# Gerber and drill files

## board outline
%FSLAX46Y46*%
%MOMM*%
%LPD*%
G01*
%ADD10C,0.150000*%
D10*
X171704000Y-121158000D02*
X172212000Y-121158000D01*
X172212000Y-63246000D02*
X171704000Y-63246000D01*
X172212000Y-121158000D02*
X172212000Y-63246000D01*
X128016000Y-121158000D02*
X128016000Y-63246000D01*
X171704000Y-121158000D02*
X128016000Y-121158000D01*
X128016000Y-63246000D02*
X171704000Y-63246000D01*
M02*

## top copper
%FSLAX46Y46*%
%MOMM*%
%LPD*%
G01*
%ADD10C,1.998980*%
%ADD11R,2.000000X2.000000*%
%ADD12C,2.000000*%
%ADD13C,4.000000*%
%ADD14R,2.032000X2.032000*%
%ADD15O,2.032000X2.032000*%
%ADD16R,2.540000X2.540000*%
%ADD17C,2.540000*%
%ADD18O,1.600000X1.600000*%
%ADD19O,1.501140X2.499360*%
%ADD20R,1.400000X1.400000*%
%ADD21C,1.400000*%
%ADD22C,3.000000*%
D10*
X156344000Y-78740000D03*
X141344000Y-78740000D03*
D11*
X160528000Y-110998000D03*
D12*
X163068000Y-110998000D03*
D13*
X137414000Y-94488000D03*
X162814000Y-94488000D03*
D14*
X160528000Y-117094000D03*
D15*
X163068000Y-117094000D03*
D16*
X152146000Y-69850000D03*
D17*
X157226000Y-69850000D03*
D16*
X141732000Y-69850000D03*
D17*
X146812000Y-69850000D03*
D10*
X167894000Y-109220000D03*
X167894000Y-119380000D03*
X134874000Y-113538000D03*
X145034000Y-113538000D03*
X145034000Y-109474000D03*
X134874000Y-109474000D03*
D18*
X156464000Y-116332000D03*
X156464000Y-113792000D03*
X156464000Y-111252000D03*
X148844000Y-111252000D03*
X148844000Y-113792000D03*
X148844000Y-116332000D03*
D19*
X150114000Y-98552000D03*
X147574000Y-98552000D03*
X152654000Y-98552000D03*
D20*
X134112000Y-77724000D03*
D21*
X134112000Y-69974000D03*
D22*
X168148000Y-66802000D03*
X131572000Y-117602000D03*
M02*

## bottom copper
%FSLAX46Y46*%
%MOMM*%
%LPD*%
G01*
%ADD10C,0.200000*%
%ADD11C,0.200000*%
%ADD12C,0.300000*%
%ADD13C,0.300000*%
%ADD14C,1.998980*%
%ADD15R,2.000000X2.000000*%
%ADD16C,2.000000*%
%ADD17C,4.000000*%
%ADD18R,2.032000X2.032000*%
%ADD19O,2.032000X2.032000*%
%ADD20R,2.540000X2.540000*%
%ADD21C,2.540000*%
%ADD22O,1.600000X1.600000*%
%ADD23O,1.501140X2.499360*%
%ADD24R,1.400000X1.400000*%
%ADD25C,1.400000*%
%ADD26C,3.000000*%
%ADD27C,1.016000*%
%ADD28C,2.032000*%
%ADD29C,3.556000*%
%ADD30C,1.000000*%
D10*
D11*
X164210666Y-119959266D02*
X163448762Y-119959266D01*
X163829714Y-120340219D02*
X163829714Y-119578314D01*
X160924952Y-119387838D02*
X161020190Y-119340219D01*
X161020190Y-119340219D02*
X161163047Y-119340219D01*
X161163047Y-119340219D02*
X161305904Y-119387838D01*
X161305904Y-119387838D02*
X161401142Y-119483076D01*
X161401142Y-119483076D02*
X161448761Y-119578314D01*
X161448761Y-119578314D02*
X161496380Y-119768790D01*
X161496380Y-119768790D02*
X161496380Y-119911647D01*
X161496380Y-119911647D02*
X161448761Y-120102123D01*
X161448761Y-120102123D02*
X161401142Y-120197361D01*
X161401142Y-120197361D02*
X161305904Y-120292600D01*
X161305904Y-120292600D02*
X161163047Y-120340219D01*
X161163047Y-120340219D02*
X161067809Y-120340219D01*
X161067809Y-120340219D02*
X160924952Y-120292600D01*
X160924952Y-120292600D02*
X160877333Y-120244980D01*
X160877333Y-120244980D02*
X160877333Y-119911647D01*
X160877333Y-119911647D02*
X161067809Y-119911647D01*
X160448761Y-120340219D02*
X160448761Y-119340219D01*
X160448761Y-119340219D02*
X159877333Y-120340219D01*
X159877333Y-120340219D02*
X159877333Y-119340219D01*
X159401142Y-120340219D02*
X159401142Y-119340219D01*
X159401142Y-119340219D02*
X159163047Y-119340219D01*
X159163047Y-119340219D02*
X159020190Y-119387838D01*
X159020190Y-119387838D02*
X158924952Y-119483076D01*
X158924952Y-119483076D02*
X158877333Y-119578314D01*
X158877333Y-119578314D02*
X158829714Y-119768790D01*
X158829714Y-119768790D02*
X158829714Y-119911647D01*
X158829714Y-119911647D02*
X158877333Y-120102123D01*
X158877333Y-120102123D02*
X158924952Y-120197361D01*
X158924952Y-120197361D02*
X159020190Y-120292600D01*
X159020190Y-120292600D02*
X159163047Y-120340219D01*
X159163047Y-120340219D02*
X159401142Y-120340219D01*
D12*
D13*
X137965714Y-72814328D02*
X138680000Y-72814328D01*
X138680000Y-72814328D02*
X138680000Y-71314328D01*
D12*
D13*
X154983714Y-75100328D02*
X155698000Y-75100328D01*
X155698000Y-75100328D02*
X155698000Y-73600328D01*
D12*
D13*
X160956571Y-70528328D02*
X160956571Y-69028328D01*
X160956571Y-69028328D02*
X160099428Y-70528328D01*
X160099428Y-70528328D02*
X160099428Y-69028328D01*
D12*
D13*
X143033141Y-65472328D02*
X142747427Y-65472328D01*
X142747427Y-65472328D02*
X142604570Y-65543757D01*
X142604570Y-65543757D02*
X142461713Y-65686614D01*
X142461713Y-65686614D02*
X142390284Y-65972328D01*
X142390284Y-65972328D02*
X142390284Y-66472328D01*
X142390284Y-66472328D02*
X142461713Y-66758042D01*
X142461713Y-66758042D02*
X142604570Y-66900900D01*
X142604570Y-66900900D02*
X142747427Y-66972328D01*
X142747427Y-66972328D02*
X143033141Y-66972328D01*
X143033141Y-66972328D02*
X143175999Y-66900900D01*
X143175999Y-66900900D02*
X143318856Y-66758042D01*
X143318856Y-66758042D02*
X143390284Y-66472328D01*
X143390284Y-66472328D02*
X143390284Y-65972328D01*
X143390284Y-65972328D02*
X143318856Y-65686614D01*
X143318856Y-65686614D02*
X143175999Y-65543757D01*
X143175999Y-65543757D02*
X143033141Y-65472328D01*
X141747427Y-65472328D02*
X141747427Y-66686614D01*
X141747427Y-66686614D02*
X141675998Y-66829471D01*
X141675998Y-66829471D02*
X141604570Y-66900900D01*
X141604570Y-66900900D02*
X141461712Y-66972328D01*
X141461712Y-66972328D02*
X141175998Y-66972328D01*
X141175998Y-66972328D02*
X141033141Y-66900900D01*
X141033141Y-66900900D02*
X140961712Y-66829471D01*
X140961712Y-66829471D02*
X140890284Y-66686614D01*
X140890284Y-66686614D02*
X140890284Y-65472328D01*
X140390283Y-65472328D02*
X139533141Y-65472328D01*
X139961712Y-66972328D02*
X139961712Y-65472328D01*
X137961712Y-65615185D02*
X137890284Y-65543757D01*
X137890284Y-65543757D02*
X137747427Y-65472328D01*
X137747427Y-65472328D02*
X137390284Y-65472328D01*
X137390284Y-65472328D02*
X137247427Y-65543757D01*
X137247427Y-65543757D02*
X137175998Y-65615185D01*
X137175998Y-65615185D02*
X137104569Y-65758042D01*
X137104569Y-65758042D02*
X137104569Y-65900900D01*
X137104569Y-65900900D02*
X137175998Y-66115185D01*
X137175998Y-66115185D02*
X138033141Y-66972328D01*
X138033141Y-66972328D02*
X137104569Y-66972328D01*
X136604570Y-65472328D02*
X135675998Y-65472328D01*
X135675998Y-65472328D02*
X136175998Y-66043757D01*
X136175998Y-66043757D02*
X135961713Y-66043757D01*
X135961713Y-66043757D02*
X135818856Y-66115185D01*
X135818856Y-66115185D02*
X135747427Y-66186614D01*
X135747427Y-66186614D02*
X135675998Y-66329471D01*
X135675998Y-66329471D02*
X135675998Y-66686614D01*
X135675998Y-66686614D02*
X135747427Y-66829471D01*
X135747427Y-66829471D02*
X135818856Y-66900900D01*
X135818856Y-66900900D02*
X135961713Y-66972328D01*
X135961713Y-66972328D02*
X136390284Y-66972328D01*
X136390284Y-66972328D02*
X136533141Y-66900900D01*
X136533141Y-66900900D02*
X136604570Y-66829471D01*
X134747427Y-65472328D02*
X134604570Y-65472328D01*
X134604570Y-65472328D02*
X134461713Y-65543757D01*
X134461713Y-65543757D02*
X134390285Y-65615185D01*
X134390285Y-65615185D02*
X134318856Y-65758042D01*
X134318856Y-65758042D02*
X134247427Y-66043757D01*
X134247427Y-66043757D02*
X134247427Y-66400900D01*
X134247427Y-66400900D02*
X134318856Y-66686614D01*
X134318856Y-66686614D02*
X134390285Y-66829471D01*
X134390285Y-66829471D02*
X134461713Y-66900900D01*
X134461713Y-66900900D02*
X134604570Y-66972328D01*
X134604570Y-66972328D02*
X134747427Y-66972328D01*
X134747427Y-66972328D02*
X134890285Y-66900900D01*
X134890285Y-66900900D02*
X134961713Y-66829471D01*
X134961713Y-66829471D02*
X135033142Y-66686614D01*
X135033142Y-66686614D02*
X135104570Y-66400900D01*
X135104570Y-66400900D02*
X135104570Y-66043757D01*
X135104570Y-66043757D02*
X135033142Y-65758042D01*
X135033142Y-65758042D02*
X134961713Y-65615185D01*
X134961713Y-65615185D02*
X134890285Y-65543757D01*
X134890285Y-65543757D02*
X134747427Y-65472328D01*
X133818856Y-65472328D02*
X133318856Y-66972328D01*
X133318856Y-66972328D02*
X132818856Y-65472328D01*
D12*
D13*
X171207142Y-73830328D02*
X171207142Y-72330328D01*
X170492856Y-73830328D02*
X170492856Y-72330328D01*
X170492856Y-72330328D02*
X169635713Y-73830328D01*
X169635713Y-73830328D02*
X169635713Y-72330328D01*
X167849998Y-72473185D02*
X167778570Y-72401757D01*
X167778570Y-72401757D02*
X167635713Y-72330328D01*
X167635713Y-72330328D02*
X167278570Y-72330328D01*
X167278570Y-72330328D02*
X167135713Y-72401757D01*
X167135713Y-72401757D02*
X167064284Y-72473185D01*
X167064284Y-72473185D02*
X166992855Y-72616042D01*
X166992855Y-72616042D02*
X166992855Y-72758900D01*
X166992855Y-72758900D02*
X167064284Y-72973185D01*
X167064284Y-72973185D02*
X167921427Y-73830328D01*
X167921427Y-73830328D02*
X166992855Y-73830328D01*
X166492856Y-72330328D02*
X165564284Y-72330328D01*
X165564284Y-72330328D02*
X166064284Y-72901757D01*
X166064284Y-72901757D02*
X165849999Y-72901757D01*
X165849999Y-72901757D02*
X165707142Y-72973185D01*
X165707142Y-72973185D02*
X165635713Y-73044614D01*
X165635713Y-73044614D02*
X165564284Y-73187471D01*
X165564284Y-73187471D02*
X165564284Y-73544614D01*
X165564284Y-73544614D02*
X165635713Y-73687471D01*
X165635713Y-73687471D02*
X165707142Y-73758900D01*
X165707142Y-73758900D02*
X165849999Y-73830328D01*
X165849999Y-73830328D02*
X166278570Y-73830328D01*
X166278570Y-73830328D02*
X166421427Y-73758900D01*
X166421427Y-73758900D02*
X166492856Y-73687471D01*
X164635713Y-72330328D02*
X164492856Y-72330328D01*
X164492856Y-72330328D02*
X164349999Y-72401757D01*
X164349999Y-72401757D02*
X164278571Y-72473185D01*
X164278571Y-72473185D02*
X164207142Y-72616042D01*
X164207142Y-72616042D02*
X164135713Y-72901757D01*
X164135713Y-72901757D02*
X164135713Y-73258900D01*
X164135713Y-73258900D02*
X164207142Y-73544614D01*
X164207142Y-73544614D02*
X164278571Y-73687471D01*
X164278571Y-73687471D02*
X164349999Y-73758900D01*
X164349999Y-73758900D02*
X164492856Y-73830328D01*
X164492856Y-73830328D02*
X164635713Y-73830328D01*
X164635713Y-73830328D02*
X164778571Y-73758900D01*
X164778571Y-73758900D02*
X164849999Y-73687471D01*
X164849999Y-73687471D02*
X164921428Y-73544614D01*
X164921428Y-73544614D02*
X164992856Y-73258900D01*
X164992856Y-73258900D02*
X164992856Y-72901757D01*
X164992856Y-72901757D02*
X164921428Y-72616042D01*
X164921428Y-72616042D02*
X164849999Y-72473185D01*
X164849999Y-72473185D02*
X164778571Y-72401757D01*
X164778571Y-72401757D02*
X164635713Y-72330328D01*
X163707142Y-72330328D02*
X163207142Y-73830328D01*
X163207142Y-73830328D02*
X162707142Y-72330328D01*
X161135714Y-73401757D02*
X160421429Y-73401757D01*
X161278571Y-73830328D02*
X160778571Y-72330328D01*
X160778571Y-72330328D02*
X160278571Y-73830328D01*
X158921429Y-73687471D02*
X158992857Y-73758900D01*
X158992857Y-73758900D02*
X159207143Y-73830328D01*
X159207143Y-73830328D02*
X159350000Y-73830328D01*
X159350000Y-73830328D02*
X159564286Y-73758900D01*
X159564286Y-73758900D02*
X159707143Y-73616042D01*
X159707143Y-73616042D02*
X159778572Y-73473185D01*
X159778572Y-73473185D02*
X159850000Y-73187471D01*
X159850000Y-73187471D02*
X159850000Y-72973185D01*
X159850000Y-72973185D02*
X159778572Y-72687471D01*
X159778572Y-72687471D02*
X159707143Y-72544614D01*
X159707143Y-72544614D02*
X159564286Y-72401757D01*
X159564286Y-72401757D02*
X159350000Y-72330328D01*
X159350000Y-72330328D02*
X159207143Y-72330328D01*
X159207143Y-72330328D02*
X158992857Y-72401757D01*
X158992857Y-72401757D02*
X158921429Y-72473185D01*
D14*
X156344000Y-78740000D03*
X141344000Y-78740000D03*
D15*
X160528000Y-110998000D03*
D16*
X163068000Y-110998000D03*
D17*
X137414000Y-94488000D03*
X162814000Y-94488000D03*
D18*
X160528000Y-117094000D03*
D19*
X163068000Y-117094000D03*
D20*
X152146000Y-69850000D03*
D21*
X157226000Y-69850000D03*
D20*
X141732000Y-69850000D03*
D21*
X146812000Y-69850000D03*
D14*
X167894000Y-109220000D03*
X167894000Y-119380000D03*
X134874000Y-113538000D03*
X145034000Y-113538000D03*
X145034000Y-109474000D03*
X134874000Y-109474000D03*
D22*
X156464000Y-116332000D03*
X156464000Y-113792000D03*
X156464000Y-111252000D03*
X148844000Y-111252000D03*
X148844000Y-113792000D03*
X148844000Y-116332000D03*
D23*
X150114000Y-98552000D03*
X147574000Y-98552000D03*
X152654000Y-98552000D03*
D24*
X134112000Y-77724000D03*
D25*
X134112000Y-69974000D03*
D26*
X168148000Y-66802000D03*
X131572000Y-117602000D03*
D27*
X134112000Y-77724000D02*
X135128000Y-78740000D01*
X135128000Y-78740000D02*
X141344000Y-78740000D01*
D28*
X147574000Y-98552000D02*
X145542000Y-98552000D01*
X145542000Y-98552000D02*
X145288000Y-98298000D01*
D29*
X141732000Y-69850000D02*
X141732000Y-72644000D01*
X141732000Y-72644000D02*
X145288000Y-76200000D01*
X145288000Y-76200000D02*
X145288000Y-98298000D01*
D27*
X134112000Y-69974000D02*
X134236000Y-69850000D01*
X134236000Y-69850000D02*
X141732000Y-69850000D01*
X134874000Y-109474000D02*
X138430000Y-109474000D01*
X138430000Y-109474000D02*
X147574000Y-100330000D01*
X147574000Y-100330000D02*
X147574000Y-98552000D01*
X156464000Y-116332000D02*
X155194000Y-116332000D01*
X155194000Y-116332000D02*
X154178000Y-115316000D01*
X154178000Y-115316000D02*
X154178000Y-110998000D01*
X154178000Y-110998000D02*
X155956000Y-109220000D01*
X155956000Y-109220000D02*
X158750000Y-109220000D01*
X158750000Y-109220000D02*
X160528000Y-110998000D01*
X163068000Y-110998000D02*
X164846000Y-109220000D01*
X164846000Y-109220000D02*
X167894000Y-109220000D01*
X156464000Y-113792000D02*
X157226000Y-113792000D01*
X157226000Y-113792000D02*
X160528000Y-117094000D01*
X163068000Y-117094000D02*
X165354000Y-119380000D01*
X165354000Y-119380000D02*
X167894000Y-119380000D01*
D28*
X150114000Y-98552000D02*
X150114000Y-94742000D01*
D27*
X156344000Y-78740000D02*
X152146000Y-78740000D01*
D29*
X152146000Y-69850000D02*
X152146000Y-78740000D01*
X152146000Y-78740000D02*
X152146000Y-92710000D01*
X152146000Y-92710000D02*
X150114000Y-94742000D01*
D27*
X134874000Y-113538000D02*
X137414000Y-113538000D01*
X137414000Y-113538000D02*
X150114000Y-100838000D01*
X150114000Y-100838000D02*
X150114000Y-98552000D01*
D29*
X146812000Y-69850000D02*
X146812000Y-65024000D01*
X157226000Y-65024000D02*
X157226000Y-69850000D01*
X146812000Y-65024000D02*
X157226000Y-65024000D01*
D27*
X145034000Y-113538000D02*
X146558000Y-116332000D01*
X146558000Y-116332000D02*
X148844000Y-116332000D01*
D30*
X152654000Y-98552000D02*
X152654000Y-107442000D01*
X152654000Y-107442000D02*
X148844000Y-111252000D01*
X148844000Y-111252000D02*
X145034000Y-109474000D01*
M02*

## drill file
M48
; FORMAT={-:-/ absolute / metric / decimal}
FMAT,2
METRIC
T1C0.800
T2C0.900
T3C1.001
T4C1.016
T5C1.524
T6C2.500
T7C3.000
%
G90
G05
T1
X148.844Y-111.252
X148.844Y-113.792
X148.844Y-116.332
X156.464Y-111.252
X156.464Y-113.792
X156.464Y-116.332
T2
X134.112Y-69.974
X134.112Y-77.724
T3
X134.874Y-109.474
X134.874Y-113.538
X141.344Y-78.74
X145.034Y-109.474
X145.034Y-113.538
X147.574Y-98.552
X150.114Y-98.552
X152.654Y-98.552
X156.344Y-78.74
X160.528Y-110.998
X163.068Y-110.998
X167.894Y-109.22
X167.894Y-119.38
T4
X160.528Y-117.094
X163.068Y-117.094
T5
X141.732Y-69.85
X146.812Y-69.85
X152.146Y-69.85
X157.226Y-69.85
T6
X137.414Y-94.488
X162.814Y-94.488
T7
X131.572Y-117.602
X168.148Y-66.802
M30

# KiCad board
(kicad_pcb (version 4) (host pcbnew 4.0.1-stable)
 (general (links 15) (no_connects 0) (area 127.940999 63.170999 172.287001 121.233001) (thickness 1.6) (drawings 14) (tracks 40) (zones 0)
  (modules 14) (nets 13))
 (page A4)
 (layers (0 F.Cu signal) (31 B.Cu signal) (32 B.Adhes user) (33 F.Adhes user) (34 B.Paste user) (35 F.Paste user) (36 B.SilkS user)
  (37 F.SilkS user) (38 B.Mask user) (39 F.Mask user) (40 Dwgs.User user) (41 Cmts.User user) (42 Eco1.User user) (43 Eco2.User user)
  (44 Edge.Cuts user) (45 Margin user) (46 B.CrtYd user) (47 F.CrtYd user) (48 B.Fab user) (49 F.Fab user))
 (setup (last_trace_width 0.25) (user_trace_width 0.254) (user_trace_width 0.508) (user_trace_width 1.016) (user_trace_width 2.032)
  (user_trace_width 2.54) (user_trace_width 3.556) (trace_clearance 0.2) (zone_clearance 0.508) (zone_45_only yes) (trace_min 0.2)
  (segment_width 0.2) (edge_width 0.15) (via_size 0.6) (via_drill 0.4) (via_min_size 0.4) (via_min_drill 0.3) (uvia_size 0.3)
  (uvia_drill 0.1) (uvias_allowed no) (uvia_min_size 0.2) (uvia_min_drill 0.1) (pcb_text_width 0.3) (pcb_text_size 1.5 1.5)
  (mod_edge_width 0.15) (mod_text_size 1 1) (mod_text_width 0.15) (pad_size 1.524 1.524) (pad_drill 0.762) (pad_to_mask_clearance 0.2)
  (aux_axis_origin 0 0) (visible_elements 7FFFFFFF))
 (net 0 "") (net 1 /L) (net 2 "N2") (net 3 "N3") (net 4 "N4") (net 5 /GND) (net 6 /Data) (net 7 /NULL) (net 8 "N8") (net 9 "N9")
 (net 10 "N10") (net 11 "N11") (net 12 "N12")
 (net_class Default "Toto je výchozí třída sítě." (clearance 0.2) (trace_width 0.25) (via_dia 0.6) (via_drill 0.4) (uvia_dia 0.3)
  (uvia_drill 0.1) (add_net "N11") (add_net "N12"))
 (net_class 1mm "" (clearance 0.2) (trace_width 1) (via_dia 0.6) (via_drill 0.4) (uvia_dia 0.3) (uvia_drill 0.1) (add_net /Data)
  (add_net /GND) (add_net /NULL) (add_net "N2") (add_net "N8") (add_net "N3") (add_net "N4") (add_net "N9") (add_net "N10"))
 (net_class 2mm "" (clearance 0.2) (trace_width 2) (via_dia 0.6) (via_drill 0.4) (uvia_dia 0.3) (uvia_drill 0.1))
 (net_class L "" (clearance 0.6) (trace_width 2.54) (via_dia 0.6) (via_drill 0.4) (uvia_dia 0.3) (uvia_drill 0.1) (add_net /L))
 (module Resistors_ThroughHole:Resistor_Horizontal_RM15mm (layer F.Cu) (at 148.844 78.74 180)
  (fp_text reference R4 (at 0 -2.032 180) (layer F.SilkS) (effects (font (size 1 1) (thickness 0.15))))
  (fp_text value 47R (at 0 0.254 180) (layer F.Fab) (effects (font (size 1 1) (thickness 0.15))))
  (pad 1 thru_hole circle (at -7.5 0 180) (size 1.99898 1.99898) (drill 1.00076) (layers *.Cu *.SilkS *.Mask) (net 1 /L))
  (pad 2 thru_hole circle (at 7.5 0 180) (size 1.99898 1.99898) (drill 1.00076) (layers *.Cu *.SilkS *.Mask) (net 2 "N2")))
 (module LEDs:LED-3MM (layer F.Cu) (at 160.528 110.998)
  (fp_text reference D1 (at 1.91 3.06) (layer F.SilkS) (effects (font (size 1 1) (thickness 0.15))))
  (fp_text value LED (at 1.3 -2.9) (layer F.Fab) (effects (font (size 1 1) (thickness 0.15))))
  (pad 1 thru_hole rect (at 0 0 90) (size 2 2) (drill 1.00076) (layers *.Cu *.Mask F.SilkS) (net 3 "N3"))
  (pad 2 thru_hole circle (at 2.54 0) (size 2 2) (drill 1.00076) (layers *.Cu *.Mask F.SilkS) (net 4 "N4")))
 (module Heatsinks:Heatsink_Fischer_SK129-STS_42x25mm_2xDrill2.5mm (layer F.Cu) (at 150.114 94.488)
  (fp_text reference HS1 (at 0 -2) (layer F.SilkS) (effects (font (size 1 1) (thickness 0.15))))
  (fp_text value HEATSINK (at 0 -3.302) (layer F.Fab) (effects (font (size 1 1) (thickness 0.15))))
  (pad 1 thru_hole circle (at -12.7 0) (size 4 4) (drill 2.5) (layers *.Cu *.Mask F.SilkS))
  (pad 1 thru_hole circle (at 12.7 0) (size 4 4) (drill 2.5) (layers *.Cu *.Mask F.SilkS)))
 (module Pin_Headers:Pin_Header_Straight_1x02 (layer F.Cu) (at 160.528 117.094 90)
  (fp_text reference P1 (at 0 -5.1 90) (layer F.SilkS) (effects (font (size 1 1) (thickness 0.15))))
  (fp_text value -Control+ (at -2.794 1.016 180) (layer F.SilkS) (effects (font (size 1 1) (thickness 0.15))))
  (pad 1 thru_hole rect (at 0 0 90) (size 2.032 2.032) (drill 1.016) (layers *.Cu *.Mask F.SilkS) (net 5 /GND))
  (pad 2 thru_hole oval (at 0 2.54 90) (size 2.032 2.032) (drill 1.016) (layers *.Cu *.Mask F.SilkS) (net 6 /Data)))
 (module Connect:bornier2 (layer F.Cu) (at 154.686 69.85)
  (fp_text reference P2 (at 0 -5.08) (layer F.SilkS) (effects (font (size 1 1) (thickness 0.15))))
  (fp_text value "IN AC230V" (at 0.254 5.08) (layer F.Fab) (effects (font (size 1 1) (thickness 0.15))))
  (pad 1 thru_hole rect (at -2.54 0) (size 2.54 2.54) (drill 1.524) (layers *.Cu *.Mask F.SilkS) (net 1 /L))
  (pad 2 thru_hole circle (at 2.54 0) (size 2.54 2.54) (drill 1.524) (layers *.Cu *.Mask F.SilkS) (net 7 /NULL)))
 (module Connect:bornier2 (layer F.Cu) (at 144.272 69.85)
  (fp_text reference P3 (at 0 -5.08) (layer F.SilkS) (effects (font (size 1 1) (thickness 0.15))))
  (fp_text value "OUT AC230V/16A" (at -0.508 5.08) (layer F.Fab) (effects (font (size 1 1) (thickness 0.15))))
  (pad 1 thru_hole rect (at -2.54 0) (size 2.54 2.54) (drill 1.524) (layers *.Cu *.Mask F.SilkS) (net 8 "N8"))
  (pad 2 thru_hole circle (at 2.54 0) (size 2.54 2.54) (drill 1.524) (layers *.Cu *.Mask F.SilkS) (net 7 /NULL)))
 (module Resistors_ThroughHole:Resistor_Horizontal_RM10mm (layer F.Cu) (at 167.894 114.3 270)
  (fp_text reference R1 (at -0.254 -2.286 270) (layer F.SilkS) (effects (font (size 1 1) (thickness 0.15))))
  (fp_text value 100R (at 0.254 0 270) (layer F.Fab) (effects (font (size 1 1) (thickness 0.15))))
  (pad 1 thru_hole circle (at -5.08 0 270) (size 1.99898 1.99898) (drill 1.00076) (layers *.Cu *.SilkS *.Mask) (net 4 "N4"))
  (pad 2 thru_hole circle (at 5.08 0 270) (size 1.99898 1.99898) (drill 1.00076) (layers *.Cu *.SilkS *.Mask) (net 6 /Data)))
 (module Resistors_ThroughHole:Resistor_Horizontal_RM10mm (layer F.Cu) (at 139.954 113.538)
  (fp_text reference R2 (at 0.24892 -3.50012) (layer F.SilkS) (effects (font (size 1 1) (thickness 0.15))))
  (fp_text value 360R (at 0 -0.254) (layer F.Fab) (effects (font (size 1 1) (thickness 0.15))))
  (pad 1 thru_hole circle (at -5.08 0) (size 1.99898 1.99898) (drill 1.00076) (layers *.Cu *.SilkS *.Mask) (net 1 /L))
  (pad 2 thru_hole circle (at 5.08 0) (size 1.99898 1.99898) (drill 1.00076) (layers *.Cu *.SilkS *.Mask) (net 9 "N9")))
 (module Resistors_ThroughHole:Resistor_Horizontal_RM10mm (layer F.Cu) (at 139.954 109.474 180)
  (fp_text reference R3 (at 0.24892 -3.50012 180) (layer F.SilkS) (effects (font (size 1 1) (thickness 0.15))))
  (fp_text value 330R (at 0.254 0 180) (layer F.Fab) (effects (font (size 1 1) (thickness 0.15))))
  (pad 1 thru_hole circle (at -5.08 0 180) (size 1.99898 1.99898) (drill 1.00076) (layers *.Cu *.SilkS *.Mask) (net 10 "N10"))
  (pad 2 thru_hole circle (at 5.08 0 180) (size 1.99898 1.99898) (drill 1.00076) (layers *.Cu *.SilkS *.Mask) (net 8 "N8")))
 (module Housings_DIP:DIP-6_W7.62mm (layer F.Cu) (at 156.464 116.332 180)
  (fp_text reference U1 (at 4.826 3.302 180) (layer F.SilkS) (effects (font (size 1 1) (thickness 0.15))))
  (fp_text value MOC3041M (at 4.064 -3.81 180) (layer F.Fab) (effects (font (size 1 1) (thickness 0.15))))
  (pad 1 thru_hole oval (at 0 0 180) (size 1.6 1.6) (drill 0.8) (layers *.Cu *.Mask F.SilkS) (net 3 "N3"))
  (pad 2 thru_hole oval (at 0 2.54 180) (size 1.6 1.6) (drill 0.8) (layers *.Cu *.Mask F.SilkS) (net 5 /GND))
  (pad 3 thru_hole oval (at 0 5.08 180) (size 1.6 1.6) (drill 0.8) (layers *.Cu *.Mask F.SilkS))
  (pad 4 thru_hole oval (at 7.62 5.08 180) (size 1.6 1.6) (drill 0.8) (layers *.Cu *.Mask F.SilkS) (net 10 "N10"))
  (pad 5 thru_hole oval (at 7.62 2.54 180) (size 1.6 1.6) (drill 0.8) (layers *.Cu *.Mask F.SilkS))
  (pad 6 thru_hole oval (at 7.62 0 180) (size 1.6 1.6) (drill 0.8) (layers *.Cu *.Mask F.SilkS) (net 9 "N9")))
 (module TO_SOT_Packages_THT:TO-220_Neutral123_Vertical (layer F.Cu) (at 150.114 98.552)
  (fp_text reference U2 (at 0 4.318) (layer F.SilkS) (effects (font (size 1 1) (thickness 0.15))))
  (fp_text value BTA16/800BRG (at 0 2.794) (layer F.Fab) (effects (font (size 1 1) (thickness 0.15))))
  (pad 2 thru_hole oval (at 0 0 90) (size 2.49936 1.50114) (drill 1.00076) (layers *.Cu *.Mask F.SilkS) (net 1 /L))
  (pad 1 thru_hole oval (at -2.54 0 90) (size 2.49936 1.50114) (drill 1.00076) (layers *.Cu *.Mask F.SilkS) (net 8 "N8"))
  (pad 3 thru_hole oval (at 2.54 0 90) (size 2.49936 1.50114) (drill 1.00076) (layers *.Cu *.Mask F.SilkS) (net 10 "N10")))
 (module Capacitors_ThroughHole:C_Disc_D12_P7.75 (layer F.Cu) (at 134.112 77.724 90)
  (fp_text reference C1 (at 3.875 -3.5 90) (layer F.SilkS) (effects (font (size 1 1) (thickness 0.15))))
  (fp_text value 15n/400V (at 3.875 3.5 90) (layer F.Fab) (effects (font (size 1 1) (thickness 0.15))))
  (pad 1 thru_hole rect (at 0 0 90) (size 1.4 1.4) (drill 0.9) (layers *.Cu *.Mask F.SilkS) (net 2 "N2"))
  (pad 2 thru_hole circle (at 7.75 0 90) (size 1.4 1.4) (drill 0.9) (layers *.Cu *.Mask F.SilkS) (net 8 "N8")))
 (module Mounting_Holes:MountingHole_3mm (layer F.Cu) (at 168.148 66.802)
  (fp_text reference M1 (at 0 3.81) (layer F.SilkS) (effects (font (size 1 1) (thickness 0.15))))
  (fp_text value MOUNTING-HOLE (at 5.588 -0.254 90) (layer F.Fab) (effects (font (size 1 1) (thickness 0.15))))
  (pad 1 thru_hole circle (at 0 0) (size 3 3) (drill 3) (layers) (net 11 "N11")))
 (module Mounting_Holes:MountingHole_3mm (layer F.Cu) (at 131.572 117.602)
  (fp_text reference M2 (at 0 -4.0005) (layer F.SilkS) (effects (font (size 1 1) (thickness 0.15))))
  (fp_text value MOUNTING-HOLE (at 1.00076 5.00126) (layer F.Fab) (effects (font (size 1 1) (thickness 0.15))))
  (pad 1 thru_hole circle (at 0 0) (size 3 3) (drill 3) (layers) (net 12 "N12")))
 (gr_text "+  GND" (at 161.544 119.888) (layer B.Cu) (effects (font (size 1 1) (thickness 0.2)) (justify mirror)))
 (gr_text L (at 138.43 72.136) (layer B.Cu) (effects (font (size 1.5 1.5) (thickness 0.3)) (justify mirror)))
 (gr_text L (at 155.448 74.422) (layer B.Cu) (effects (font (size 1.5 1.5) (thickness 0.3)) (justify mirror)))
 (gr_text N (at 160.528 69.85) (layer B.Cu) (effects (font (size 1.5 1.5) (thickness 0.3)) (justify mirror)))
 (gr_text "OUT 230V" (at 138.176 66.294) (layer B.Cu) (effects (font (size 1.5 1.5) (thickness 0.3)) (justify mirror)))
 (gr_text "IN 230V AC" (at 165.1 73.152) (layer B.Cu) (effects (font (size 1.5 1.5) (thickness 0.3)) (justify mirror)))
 (gr_line (start 171.704 121.158) (end 172.212 121.158) (angle 90) (layer Edge.Cuts) (width 0.15))
 (gr_line (start 172.212 63.246) (end 171.704 63.246) (angle 90) (layer Edge.Cuts) (width 0.15))
 (gr_line (start 172.212 121.158) (end 172.212 63.246) (angle 90) (layer Edge.Cuts) (width 0.15))
 (gr_line (start 128.016 121.158) (end 128.016 63.246) (angle 90) (layer Edge.Cuts) (width 0.15))
 (gr_line (start 171.704 121.158) (end 128.016 121.158) (angle 90) (layer Edge.Cuts) (width 0.15))
 (gr_line (start 128.016 63.246) (end 171.704 63.246) (angle 90) (layer Edge.Cuts) (width 0.15))
 (segment (start 134.112 77.724) (end 135.128 78.74) (width 1.016) (layer B.Cu) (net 2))
 (segment (start 135.128 78.74) (end 141.344 78.74) (width 1.016) (layer B.Cu) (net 2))
 (segment (start 147.574 98.552) (end 145.542 98.552) (width 2.032) (layer B.Cu) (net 8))
 (segment (start 145.542 98.552) (end 145.288 98.298) (width 2.032) (layer B.Cu) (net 8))
 (segment (start 141.732 69.85) (end 141.732 72.644) (width 3.556) (layer B.Cu) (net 8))
 (segment (start 141.732 72.644) (end 145.288 76.2) (width 3.556) (layer B.Cu) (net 8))
 (segment (start 145.288 76.2) (end 145.288 98.298) (width 3.556) (layer B.Cu) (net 8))
 (segment (start 134.112 69.974) (end 134.236 69.85) (width 1.016) (layer B.Cu) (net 8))
 (segment (start 134.236 69.85) (end 141.732 69.85) (width 1.016) (layer B.Cu) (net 8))
 (segment (start 134.874 109.474) (end 138.43 109.474) (width 1.016) (layer B.Cu) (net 8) (status 10))
 (segment (start 138.43 109.474) (end 147.574 100.33) (width 1.016) (layer B.Cu) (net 8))
 (segment (start 147.574 100.33) (end 147.574 98.552) (width 1.016) (layer B.Cu) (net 8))
 (segment (start 156.464 116.332) (end 155.194 116.332) (width 1.016) (layer B.Cu) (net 3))
 (segment (start 155.194 116.332) (end 154.178 115.316) (width 1.016) (layer B.Cu) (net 3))
 (segment (start 154.178 115.316) (end 154.178 110.998) (width 1.016) (layer B.Cu) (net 3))
 (segment (start 154.178 110.998) (end 155.956 109.22) (width 1.016) (layer B.Cu) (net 3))
 (segment (start 155.956 109.22) (end 158.75 109.22) (width 1.016) (layer B.Cu) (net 3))
 (segment (start 158.75 109.22) (end 160.528 110.998) (width 1.016) (layer B.Cu) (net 3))
 (segment (start 163.068 110.998) (end 164.846 109.22) (width 1.016) (layer B.Cu) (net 4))
 (segment (start 164.846 109.22) (end 167.894 109.22) (width 1.016) (layer B.Cu) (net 4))
 (segment (start 156.464 113.792) (end 157.226 113.792) (width 1.016) (layer B.Cu) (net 5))
 (segment (start 157.226 113.792) (end 160.528 117.094) (width 1.016) (layer B.Cu) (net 5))
 (segment (start 163.068 117.094) (end 165.354 119.38) (width 1.016) (layer B.Cu) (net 6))
 (segment (start 165.354 119.38) (end 167.894 119.38) (width 1.016) (layer B.Cu) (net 6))
 (segment (start 150.114 98.552) (end 150.114 94.742) (width 2.032) (layer B.Cu) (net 1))
 (segment (start 156.344 78.74) (end 152.146 78.74) (width 1.016) (layer B.Cu) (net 1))
 (segment (start 152.146 69.85) (end 152.146 78.74) (width 3.556) (layer B.Cu) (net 1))
 (segment (start 152.146 78.74) (end 152.146 92.71) (width 3.556) (layer B.Cu) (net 1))
 (segment (start 152.146 92.71) (end 150.114 94.742) (width 3.556) (layer B.Cu) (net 1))
 (segment (start 134.874 113.538) (end 137.414 113.538) (width 1.016) (layer B.Cu) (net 1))
 (segment (start 137.414 113.538) (end 150.114 100.838) (width 1.016) (layer B.Cu) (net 1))
 (segment (start 150.114 100.838) (end 150.114 98.552) (width 1.016) (layer B.Cu) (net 1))
 (segment (start 146.812 69.85) (end 146.812 65.024) (width 3.556) (layer B.Cu) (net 7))
 (segment (start 157.226 65.024) (end 157.226 69.85) (width 3.556) (layer B.Cu) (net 7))
 (segment (start 146.812 65.024) (end 157.226 65.024) (width 3.556) (layer B.Cu) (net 7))
 (segment (start 145.034 113.538) (end 146.558 116.332) (width 1.016) (layer B.Cu) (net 9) (status 10))
 (segment (start 146.558 116.332) (end 148.844 116.332) (width 1.016) (layer B.Cu) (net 9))
 (segment (start 152.654 98.552) (end 152.654 107.442) (width 1) (layer B.Cu) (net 10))
 (segment (start 152.654 107.442) (end 148.844 111.252) (width 1) (layer B.Cu) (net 10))
 (segment (start 148.844 111.252) (end 145.034 109.474) (width 1) (layer B.Cu) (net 10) (status 20)))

